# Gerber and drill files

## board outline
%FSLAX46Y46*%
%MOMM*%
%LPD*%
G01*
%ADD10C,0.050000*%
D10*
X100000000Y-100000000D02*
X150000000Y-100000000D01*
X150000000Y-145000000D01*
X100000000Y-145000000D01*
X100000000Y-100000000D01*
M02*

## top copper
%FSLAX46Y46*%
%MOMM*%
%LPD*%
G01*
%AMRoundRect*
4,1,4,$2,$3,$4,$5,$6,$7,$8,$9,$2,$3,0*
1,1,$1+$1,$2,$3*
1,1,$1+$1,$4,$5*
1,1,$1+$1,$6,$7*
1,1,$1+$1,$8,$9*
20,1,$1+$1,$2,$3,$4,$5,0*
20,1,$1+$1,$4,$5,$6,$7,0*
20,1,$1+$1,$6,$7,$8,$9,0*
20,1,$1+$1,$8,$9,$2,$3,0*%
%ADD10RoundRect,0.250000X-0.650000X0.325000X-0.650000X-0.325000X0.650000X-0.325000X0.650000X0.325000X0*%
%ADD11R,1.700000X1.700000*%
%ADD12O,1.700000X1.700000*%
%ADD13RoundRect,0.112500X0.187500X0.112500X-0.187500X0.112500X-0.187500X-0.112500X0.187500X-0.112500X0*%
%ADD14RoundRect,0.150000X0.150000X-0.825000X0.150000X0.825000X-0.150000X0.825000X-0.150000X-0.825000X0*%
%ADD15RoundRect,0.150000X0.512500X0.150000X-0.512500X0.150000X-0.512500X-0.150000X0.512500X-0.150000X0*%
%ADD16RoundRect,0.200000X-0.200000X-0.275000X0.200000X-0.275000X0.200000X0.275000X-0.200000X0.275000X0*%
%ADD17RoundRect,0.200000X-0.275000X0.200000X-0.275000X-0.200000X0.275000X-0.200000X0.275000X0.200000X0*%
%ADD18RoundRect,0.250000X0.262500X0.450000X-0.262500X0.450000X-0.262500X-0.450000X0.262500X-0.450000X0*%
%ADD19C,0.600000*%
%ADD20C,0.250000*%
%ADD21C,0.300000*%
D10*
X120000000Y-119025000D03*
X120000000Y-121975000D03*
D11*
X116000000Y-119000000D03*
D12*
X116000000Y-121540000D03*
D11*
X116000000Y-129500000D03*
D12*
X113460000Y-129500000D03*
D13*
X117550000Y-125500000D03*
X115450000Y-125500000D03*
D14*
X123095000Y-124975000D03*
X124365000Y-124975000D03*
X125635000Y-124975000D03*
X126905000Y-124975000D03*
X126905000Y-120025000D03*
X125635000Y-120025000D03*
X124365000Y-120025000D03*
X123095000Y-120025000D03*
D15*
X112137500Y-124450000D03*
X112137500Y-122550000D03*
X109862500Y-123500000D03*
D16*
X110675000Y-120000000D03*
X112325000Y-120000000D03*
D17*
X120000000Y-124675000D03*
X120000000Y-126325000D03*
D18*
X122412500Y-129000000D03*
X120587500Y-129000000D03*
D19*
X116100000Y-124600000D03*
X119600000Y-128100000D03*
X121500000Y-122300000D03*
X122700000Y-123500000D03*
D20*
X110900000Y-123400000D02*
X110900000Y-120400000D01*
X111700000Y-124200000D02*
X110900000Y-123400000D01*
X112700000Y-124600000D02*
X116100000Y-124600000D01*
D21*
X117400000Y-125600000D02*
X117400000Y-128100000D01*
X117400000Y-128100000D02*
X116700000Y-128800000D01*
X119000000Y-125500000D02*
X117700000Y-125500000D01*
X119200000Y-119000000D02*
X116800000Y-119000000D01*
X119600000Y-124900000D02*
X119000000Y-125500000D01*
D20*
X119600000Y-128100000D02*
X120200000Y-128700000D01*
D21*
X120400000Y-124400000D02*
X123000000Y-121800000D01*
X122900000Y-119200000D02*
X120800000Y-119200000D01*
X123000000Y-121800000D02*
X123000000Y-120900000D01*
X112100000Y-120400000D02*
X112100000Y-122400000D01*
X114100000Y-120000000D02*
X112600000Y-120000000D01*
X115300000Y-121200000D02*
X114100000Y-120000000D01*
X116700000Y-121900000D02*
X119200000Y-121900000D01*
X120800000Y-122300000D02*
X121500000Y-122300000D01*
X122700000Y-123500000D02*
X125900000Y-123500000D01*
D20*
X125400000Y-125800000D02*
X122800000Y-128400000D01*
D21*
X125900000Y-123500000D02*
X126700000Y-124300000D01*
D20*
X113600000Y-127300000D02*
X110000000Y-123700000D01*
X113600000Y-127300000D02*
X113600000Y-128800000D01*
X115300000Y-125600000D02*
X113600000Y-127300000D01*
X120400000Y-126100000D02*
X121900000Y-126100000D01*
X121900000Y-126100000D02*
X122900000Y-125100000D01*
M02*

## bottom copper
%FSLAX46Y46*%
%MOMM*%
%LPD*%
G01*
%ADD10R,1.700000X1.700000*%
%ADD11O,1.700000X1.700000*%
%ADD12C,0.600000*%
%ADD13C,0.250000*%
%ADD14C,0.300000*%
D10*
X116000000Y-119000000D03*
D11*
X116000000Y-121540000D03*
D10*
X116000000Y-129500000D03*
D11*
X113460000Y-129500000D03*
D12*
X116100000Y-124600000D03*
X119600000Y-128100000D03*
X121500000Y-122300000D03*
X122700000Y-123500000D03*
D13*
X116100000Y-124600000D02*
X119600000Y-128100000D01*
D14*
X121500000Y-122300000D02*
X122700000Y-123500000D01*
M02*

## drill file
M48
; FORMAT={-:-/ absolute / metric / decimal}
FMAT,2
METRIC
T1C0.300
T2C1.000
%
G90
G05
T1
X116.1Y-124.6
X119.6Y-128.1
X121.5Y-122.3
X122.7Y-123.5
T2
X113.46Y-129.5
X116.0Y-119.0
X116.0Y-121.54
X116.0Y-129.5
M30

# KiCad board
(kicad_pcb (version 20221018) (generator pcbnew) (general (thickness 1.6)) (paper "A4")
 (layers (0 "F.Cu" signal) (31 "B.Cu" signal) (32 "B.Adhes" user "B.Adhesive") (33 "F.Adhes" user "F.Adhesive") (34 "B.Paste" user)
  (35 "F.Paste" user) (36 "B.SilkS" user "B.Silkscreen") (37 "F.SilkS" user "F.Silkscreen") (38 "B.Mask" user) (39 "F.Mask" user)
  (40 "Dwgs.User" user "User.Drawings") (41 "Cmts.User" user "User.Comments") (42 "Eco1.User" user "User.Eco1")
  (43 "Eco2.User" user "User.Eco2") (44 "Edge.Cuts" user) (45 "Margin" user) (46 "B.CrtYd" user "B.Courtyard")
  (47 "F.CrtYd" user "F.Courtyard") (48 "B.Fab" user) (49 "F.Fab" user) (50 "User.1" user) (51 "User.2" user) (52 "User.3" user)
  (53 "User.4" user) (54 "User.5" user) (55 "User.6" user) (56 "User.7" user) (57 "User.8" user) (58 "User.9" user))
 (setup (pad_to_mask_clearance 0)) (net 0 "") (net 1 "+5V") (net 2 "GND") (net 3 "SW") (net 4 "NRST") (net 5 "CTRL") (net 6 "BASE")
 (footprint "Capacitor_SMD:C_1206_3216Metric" (layer "F.Cu") (at 120 120.5 -90)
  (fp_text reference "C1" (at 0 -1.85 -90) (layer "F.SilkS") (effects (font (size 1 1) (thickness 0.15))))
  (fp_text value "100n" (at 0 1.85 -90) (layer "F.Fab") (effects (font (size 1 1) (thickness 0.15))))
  (pad "1" smd roundrect (at -1.475 0 270) (size 1.15 1.8) (layers "F.Cu" "F.Paste" "F.Mask") (roundrect_rratio 0.217391) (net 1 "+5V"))
  (pad "2" smd roundrect (at 1.475 0 270) (size 1.15 1.8) (layers "F.Cu" "F.Paste" "F.Mask") (roundrect_rratio 0.217391) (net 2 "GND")))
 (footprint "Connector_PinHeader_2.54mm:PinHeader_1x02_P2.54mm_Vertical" (layer "F.Cu") (at 116 119)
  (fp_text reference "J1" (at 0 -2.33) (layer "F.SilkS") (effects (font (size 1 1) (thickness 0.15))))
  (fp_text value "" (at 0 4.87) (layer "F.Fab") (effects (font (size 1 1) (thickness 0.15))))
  (pad "1" thru_hole rect (at 0 0) (size 1.7 1.7) (drill 1) (layers "*.Cu" "*.Mask") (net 1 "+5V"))
  (pad "2" thru_hole oval (at 0 2.54) (size 1.7 1.7) (drill 1) (layers "*.Cu" "*.Mask") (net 2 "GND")))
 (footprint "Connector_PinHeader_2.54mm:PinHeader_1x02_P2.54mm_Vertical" (layer "F.Cu") (at 116 129.5 -90)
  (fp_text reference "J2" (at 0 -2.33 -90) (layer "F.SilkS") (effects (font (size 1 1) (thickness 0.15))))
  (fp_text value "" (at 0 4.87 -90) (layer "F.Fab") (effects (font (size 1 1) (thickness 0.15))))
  (pad "1" thru_hole rect (at 0 0 270) (size 1.7 1.7) (drill 1) (layers "*.Cu" "*.Mask") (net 1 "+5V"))
  (pad "2" thru_hole oval (at 0 2.54 270) (size 1.7 1.7) (drill 1) (layers "*.Cu" "*.Mask") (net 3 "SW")))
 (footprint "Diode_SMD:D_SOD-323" (layer "F.Cu") (at 116.5 125.5 180)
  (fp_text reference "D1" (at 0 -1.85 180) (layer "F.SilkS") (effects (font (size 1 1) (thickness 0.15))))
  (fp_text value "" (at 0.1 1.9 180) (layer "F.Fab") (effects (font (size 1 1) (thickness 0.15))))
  (pad "1" smd roundrect (at -1.05 0 180) (size 0.6 0.45) (layers "F.Cu" "F.Paste" "F.Mask") (roundrect_rratio 0.25) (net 1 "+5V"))
  (pad "2" smd roundrect (at 1.05 0 180) (size 0.6 0.45) (layers "F.Cu" "F.Paste" "F.Mask") (roundrect_rratio 0.25) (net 3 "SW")))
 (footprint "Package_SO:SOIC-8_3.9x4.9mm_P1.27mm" (layer "F.Cu") (at 125 122.5 90)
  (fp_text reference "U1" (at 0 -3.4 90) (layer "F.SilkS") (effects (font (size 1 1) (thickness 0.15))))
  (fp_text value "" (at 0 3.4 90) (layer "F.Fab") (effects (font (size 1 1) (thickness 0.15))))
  (pad "1" smd roundrect (at -2.475 -1.905 90) (size 1.95 0.6) (layers "F.Cu" "F.Paste" "F.Mask") (roundrect_rratio 0.25) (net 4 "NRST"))
  (pad "2" smd roundrect (at -2.475 -0.635 90) (size 1.95 0.6) (layers "F.Cu" "F.Paste" "F.Mask") (roundrect_rratio 0.25))
  (pad "3" smd roundrect (at -2.475 0.635 90) (size 1.95 0.6) (layers "F.Cu" "F.Paste" "F.Mask") (roundrect_rratio 0.25) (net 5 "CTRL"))
  (pad "4" smd roundrect (at -2.475 1.905 90) (size 1.95 0.6) (layers "F.Cu" "F.Paste" "F.Mask") (roundrect_rratio 0.25) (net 2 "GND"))
  (pad "5" smd roundrect (at 2.475 1.905 90) (size 1.95 0.6) (layers "F.Cu" "F.Paste" "F.Mask") (roundrect_rratio 0.25))
  (pad "6" smd roundrect (at 2.475 0.635 90) (size 1.95 0.6) (layers "F.Cu" "F.Paste" "F.Mask") (roundrect_rratio 0.25))
  (pad "7" smd roundrect (at 2.475 -0.635 90) (size 1.95 0.6) (layers "F.Cu" "F.Paste" "F.Mask") (roundrect_rratio 0.25))
  (pad "8" smd roundrect (at 2.475 -1.905 90) (size 1.95 0.6) (layers "F.Cu" "F.Paste" "F.Mask") (roundrect_rratio 0.25) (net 1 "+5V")))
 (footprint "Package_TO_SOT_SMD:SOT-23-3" (layer "F.Cu") (at 111 123.5 180)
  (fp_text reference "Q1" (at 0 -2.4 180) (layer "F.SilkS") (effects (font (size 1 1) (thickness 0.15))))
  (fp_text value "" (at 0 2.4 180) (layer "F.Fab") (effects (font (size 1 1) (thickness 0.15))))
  (pad "1" smd roundrect (at -1.1375 -0.95 180) (size 1.325 0.6) (layers "F.Cu" "F.Paste" "F.Mask") (roundrect_rratio 0.25) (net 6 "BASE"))
  (pad "2" smd roundrect (at -1.1375 0.95 180) (size 1.325 0.6) (layers "F.Cu" "F.Paste" "F.Mask") (roundrect_rratio 0.25) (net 2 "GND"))
  (pad "3" smd roundrect (at 1.1375 0 180) (size 1.325 0.6) (layers "F.Cu" "F.Paste" "F.Mask") (roundrect_rratio 0.25) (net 3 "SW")))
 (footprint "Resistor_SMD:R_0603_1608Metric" (layer "F.Cu") (at 111.5 120)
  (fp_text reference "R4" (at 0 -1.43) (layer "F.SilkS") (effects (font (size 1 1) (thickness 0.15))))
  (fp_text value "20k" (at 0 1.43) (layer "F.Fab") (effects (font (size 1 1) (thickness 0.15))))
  (pad "1" smd roundrect (at -0.825 0) (size 0.8 0.95) (layers "F.Cu" "F.Paste" "F.Mask") (roundrect_rratio 0.25) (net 6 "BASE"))
  (pad "2" smd roundrect (at 0.825 0) (size 0.8 0.95) (layers "F.Cu" "F.Paste" "F.Mask") (roundrect_rratio 0.25) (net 2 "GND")))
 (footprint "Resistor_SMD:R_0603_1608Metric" (layer "F.Cu") (at 120 125.5 -90)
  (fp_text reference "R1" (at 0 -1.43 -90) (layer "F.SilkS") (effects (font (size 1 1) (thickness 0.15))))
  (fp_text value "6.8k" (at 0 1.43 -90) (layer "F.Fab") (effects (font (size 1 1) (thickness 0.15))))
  (pad "1" smd roundrect (at -0.825 0 270) (size 0.8 0.95) (layers "F.Cu" "F.Paste" "F.Mask") (roundrect_rratio 0.25) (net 1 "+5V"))
  (pad "2" smd roundrect (at 0.825 0 270) (size 0.8 0.95) (layers "F.Cu" "F.Paste" "F.Mask") (roundrect_rratio 0.25) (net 4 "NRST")))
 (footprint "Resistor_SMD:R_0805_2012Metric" (layer "F.Cu") (at 121.5 129 180)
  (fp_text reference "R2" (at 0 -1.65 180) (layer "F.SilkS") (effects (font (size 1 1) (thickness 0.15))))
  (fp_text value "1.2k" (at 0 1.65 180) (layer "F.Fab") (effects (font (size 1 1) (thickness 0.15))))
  (pad "1" smd roundrect (at -0.9125 0 180) (size 1.025 1.4) (layers "F.Cu" "F.Paste" "F.Mask") (roundrect_rratio 0.243902) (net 5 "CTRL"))
  (pad "2" smd roundrect (at 0.9125 0 180) (size 1.025 1.4) (layers "F.Cu" "F.Paste" "F.Mask") (roundrect_rratio 0.243902) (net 6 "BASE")))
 (gr_rect (start 100 100) (end 150 145) (stroke (width 0.05) (type default)) (fill none) (layer "Edge.Cuts"))
 (segment (start 110.9 123.4) (end 110.9 120.4) (width 0.25) (layer "F.Cu") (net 6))
 (segment (start 111.7 124.2) (end 110.9 123.4) (width 0.25) (layer "F.Cu") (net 6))
 (segment (start 112.7 124.6) (end 116.1 124.6) (width 0.25) (layer "F.Cu") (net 6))
 (segment (start 117.4 125.6) (end 117.4 128.1) (width 0.3) (layer "F.Cu") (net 1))
 (segment (start 117.4 128.1) (end 116.7 128.8) (width 0.3) (layer "F.Cu") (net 1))
 (segment (start 119 125.5) (end 117.7 125.5) (width 0.3) (layer "F.Cu") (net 1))
 (segment (start 119.2 119) (end 116.8 119) (width 0.3) (layer "F.Cu") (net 1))
 (segment (start 119.6 124.9) (end 119 125.5) (width 0.3) (layer "F.Cu") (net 1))
 (segment (start 119.6 128.1) (end 120.2 128.7) (width 0.25) (layer "F.Cu") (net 6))
 (segment (start 120.4 124.4) (end 123 121.8) (width 0.3) (layer "F.Cu") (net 1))
 (segment (start 122.9 119.2) (end 120.8 119.2) (width 0.3) (layer "F.Cu") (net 1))
 (segment (start 123 121.8) (end 123 120.9) (width 0.3) (layer "F.Cu") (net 1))
 (via (at 116.1 124.6) (size 0.6) (drill 0.3) (layers "F.Cu" "B.Cu") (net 6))
 (via (at 119.6 128.1) (size 0.6) (drill 0.3) (layers "F.Cu" "B.Cu") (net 6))
 (segment (start 112.1 120.4) (end 112.1 122.4) (width 0.3) (layer "F.Cu") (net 2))
 (segment (start 114.1 120) (end 112.6 120) (width 0.3) (layer "F.Cu") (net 2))
 (segment (start 115.3 121.2) (end 114.1 120) (width 0.3) (layer "F.Cu") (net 2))
 (segment (start 116.1 124.6) (end 119.6 128.1) (width 0.25) (layer "B.Cu") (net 6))
 (segment (start 116.7 121.9) (end 119.2 121.9) (width 0.3) (layer "F.Cu") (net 2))
 (segment (start 120.8 122.3) (end 121.5 122.3) (width 0.3) (layer "F.Cu") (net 2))
 (segment (start 122.7 123.5) (end 125.9 123.5) (width 0.3) (layer "F.Cu") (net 2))
 (segment (start 125.4 125.8) (end 122.8 128.4) (width 0.25) (layer "F.Cu") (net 5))
 (segment (start 125.9 123.5) (end 126.7 124.3) (width 0.3) (layer "F.Cu") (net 2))
 (via (at 121.5 122.3) (size 0.6) (drill 0.3) (layers "F.Cu" "B.Cu") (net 2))
 (via (at 122.7 123.5) (size 0.6) (drill 0.3) (layers "F.Cu" "B.Cu") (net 2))
 (segment (start 113.6 127.3) (end 110 123.7) (width 0.25) (layer "F.Cu") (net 3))
 (segment (start 113.6 127.3) (end 113.6 128.8) (width 0.25) (layer "F.Cu") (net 3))
 (segment (start 115.3 125.6) (end 113.6 127.3) (width 0.25) (layer "F.Cu") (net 3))
 (segment (start 120.4 126.1) (end 121.9 126.1) (width 0.25) (layer "F.Cu") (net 4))
 (segment (start 121.5 122.3) (end 122.7 123.5) (width 0.3) (layer "B.Cu") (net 2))
 (segment (start 121.9 126.1) (end 122.9 125.1) (width 0.25) (layer "F.Cu") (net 4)))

